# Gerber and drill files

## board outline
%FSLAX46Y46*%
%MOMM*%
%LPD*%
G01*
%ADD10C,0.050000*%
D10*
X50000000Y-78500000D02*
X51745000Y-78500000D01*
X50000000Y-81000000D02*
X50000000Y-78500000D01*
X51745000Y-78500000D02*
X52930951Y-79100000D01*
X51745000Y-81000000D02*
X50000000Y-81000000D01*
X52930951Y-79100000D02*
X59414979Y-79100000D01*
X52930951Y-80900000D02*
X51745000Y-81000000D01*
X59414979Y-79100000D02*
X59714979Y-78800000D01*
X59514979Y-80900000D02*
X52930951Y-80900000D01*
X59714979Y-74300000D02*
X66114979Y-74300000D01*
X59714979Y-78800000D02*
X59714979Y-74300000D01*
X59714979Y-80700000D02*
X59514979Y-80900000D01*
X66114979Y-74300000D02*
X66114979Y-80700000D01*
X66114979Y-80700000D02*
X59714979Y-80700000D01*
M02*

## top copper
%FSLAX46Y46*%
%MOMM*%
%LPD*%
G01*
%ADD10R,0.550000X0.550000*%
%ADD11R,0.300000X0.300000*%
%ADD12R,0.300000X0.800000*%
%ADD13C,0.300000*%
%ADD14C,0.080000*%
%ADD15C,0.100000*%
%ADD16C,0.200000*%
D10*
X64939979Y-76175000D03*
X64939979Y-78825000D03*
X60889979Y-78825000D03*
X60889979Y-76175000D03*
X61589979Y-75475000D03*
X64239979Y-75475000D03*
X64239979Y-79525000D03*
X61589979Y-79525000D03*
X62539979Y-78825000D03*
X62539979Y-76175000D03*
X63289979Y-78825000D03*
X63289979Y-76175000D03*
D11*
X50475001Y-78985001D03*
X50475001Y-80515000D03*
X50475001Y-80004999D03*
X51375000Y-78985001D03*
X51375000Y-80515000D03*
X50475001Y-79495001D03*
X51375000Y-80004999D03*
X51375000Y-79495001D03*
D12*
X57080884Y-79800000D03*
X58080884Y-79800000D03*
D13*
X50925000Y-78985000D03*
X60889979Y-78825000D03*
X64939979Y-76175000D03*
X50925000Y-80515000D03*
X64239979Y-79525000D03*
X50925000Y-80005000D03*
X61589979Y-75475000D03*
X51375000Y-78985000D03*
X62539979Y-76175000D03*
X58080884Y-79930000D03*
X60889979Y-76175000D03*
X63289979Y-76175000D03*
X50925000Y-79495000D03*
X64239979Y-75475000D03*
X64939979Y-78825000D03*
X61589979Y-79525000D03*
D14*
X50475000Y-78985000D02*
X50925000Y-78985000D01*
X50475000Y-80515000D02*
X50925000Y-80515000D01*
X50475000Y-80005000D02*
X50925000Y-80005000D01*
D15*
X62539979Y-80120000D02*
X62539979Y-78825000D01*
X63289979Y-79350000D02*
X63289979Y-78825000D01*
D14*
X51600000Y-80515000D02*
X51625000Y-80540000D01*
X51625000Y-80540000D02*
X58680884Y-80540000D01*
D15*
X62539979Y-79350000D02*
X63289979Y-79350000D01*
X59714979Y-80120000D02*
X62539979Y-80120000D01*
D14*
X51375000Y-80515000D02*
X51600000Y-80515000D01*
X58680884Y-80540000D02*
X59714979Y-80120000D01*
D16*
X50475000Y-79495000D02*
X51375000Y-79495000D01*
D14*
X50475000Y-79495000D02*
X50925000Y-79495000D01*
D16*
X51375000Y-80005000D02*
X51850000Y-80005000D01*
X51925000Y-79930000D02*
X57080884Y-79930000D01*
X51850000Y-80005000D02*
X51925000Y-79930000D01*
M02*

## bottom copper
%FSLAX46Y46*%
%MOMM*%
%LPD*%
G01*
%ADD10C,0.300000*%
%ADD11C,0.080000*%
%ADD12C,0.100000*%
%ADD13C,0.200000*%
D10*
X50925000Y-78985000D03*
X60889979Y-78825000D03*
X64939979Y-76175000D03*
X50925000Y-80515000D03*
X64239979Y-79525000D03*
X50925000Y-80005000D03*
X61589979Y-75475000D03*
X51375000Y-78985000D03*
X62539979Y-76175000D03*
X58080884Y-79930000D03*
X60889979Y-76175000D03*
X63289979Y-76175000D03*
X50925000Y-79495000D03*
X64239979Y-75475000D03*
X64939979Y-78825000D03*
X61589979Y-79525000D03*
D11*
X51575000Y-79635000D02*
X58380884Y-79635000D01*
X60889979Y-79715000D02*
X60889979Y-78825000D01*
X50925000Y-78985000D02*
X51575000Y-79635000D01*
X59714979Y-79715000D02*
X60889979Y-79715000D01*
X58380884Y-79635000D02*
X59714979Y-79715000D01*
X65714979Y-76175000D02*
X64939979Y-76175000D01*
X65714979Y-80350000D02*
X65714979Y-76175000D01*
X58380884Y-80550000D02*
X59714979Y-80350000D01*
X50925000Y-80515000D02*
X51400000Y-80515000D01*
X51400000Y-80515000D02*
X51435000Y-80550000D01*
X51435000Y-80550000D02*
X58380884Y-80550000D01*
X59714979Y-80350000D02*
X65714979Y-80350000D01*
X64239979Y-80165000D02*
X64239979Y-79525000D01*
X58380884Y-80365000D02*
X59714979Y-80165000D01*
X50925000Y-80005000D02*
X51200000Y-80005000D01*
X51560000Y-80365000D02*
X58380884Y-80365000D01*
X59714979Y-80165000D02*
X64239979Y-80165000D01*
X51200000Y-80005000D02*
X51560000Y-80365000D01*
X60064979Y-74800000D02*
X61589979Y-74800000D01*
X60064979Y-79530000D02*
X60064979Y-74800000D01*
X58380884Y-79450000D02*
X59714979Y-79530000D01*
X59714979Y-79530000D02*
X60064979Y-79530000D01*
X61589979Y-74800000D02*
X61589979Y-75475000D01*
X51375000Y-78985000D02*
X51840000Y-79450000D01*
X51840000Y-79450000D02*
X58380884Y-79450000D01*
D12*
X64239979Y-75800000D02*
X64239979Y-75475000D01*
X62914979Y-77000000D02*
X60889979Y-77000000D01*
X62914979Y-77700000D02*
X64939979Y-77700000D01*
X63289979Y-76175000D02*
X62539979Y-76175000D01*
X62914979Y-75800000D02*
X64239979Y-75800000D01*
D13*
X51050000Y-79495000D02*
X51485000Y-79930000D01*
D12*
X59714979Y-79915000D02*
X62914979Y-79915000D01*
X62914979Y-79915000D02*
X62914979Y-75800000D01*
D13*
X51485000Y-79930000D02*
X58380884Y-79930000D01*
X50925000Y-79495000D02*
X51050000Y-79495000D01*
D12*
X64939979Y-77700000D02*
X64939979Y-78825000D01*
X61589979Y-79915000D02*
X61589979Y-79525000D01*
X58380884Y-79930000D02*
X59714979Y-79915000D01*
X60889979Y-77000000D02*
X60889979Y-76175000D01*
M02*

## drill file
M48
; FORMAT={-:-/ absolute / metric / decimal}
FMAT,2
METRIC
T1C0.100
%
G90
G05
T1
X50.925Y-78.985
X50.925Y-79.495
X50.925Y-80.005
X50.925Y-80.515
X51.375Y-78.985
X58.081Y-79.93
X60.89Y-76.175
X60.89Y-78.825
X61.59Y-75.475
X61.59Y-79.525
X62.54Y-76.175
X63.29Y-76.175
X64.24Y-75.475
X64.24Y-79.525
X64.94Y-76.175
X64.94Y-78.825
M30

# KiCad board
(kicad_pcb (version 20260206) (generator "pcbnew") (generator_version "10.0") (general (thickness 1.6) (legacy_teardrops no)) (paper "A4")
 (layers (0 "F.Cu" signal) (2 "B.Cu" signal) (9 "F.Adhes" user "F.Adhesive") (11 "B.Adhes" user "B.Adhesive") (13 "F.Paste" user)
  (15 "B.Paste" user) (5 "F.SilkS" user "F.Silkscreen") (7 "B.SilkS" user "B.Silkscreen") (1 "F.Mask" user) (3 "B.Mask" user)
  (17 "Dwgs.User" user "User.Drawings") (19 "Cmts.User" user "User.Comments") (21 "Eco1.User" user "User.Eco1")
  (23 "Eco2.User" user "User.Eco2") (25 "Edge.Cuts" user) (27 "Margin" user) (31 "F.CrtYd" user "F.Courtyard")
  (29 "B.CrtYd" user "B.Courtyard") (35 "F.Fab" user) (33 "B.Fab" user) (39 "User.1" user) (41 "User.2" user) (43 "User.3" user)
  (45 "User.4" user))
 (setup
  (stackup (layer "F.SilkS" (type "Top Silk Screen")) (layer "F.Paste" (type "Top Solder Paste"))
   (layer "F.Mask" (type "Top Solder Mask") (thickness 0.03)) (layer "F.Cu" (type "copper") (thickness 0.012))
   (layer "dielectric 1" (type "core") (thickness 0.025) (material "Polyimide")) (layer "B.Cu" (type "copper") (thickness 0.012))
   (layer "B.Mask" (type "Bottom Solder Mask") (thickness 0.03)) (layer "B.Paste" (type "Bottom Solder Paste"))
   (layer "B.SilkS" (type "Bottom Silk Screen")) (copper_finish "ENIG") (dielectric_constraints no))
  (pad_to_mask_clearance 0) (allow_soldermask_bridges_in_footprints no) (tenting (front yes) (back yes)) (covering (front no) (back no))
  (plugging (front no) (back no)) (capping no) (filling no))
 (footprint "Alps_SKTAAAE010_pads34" (layer "F.Cu") (at 65.314979 77.5 -90)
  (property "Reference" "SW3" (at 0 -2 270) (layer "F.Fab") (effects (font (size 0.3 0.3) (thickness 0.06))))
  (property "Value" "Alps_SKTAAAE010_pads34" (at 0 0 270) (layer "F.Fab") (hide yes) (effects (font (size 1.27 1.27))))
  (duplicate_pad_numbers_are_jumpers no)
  (pad "3" smd rect (at -1.325 0.375 270) (size 0.55 0.55) (layers "F.Cu" "F.Mask") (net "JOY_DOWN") (solder_mask_margin 0.05)
   (thermal_bridge_angle 45))
  (pad "4" smd rect (at 1.325 0.375 270) (size 0.55 0.55) (layers "F.Cu" "F.Mask") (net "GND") (solder_mask_margin 0.05)
   (thermal_bridge_angle 45)))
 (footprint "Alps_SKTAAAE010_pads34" (layer "F.Cu") (at 62.914979 79.9 180)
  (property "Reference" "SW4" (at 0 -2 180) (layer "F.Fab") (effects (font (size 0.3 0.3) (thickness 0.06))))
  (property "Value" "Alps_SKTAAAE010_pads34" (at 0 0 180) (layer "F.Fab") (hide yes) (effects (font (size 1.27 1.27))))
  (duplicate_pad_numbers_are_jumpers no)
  (pad "3" smd rect (at -1.325 0.375 180) (size 0.55 0.55) (layers "F.Cu" "F.Mask") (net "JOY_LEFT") (solder_mask_margin 0.05)
   (thermal_bridge_angle 45))
  (pad "4" smd rect (at 1.325 0.375 180) (size 0.55 0.55) (layers "F.Cu" "F.Mask") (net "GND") (solder_mask_margin 0.05)
   (thermal_bridge_angle 45)))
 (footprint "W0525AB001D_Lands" (layer "F.Cu") (at 57.580884 79.93)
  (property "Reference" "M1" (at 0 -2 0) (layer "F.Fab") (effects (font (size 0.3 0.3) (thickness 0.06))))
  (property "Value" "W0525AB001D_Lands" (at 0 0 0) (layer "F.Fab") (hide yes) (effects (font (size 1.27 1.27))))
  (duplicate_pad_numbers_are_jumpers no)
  (pad "1" smd rect (at -0.5 -0.13) (size 0.3 0.8) (layers "F.Cu" "F.Mask") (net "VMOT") (solder_mask_margin 0.05) (thermal_bridge_angle 45))
  (pad "2" smd rect (at 0.5 -0.13) (size 0.3 0.8) (layers "F.Cu" "F.Mask") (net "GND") (solder_mask_margin 0.05) (thermal_bridge_angle 45)))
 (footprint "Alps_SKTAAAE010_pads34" (layer "F.Cu") (at 60.514979 77.5 90)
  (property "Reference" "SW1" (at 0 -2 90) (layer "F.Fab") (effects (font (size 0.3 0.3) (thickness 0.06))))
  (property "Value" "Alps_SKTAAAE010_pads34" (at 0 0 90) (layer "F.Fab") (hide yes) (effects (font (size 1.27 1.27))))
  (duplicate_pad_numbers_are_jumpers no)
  (pad "3" smd rect (at -1.325 0.375 90) (size 0.55 0.55) (layers "F.Cu" "F.Mask") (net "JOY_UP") (solder_mask_margin 0.05)
   (thermal_bridge_angle 45))
  (pad "4" smd rect (at 1.325 0.375 90) (size 0.55 0.55) (layers "F.Cu" "F.Mask") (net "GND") (solder_mask_margin 0.05)
   (thermal_bridge_angle 45)))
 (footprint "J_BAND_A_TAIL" (layer "F.Cu") (at 50.9 79.75)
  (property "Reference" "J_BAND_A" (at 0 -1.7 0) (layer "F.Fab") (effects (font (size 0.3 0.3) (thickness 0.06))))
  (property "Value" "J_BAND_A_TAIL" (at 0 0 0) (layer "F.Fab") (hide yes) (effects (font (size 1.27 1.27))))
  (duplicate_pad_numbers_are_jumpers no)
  (pad "1" smd rect (at -0.424999 -0.764999) (size 0.3 0.3) (layers "F.Cu" "F.Mask") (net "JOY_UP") (solder_mask_margin 0.05)
   (thermal_bridge_angle 45))
  (pad "2" smd rect (at -0.424999 0.765) (size 0.3 0.3) (layers "F.Cu" "F.Mask") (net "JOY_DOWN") (solder_mask_margin 0.05)
   (thermal_bridge_angle 45))
  (pad "3" smd rect (at -0.424999 0.254999) (size 0.3 0.3) (layers "F.Cu" "F.Mask") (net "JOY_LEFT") (solder_mask_margin 0.05)
   (thermal_bridge_angle 45))
  (pad "4" smd rect (at 0.475 -0.764999) (size 0.3 0.3) (layers "F.Cu" "F.Mask") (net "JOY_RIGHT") (solder_mask_margin 0.05)
   (thermal_bridge_angle 45))
  (pad "5" smd rect (at 0.475 0.765) (size 0.3 0.3) (layers "F.Cu" "F.Mask") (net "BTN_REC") (solder_mask_margin 0.05)
   (thermal_bridge_angle 45))
  (pad "6" smd rect (at -0.424999 -0.254999) (size 0.3 0.3) (layers "F.Cu" "F.Mask") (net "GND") (solder_mask_margin 0.05)
   (thermal_bridge_angle 45))
  (pad "7" smd rect (at 0.475 0.254999) (size 0.3 0.3) (layers "F.Cu" "F.Mask") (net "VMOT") (solder_mask_margin 0.05)
   (thermal_bridge_angle 45))
  (pad "8" smd rect (at 0.475 -0.254999) (size 0.3 0.3) (layers "F.Cu" "F.Mask") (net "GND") (solder_mask_margin 0.05)
   (thermal_bridge_angle 45)))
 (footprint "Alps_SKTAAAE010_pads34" (layer "F.Cu") (at 62.914979 75.1)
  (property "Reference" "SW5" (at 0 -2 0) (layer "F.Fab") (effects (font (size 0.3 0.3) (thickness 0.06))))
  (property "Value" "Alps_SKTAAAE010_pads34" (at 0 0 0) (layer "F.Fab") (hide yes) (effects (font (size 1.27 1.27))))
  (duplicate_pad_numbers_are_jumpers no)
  (pad "3" smd rect (at -1.325 0.375) (size 0.55 0.55) (layers "F.Cu" "F.Mask") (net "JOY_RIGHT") (solder_mask_margin 0.05)
   (thermal_bridge_angle 45))
  (pad "4" smd rect (at 1.325 0.375) (size 0.55 0.55) (layers "F.Cu" "F.Mask") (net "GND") (solder_mask_margin 0.05)
   (thermal_bridge_angle 45)))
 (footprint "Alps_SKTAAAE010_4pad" (layer "F.Cu") (at 62.914979 77.5 90)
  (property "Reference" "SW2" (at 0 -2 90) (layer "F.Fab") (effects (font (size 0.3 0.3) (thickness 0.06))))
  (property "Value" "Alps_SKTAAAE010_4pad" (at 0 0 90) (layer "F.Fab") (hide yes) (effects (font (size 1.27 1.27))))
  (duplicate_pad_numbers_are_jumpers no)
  (pad "1" smd rect (at -1.325 -0.375 90) (size 0.55 0.55) (layers "F.Cu" "F.Mask") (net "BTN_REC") (solder_mask_margin 0.05)
   (thermal_bridge_angle 45))
  (pad "2" smd rect (at 1.325 -0.375 90) (size 0.55 0.55) (layers "F.Cu" "F.Mask") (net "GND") (solder_mask_margin 0.05)
   (thermal_bridge_angle 45))
  (pad "3" smd rect (at -1.325 0.375 90) (size 0.55 0.55) (layers "F.Cu" "F.Mask") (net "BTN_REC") (solder_mask_margin 0.05)
   (thermal_bridge_angle 45))
  (pad "4" smd rect (at 1.325 0.375 90) (size 0.55 0.55) (layers "F.Cu" "F.Mask") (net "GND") (solder_mask_margin 0.05)
   (thermal_bridge_angle 45)))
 (gr_line (start 50 78.5) (end 51.745 78.5) (stroke (width 0.05) (type default)) (layer "Edge.Cuts"))
 (gr_line (start 50 81) (end 50 78.5) (stroke (width 0.05) (type default)) (layer "Edge.Cuts"))
 (gr_line (start 51.745 78.5) (end 52.930951 79.1) (stroke (width 0.05) (type default)) (layer "Edge.Cuts"))
 (gr_line (start 51.745 81) (end 50 81) (stroke (width 0.05) (type default)) (layer "Edge.Cuts"))
 (gr_line (start 52.930951 79.1) (end 59.414979 79.1) (stroke (width 0.05) (type default)) (layer "Edge.Cuts"))
 (gr_line (start 52.930951 80.9) (end 51.745 81) (stroke (width 0.05) (type default)) (layer "Edge.Cuts"))
 (gr_line (start 59.414979 79.1) (end 59.714979 78.8) (stroke (width 0.05) (type default)) (layer "Edge.Cuts"))
 (gr_line (start 59.514979 80.9) (end 52.930951 80.9) (stroke (width 0.05) (type default)) (layer "Edge.Cuts"))
 (gr_line (start 59.714979 74.3) (end 66.114979 74.3) (stroke (width 0.05) (type default)) (layer "Edge.Cuts"))
 (gr_line (start 59.714979 78.8) (end 59.714979 74.3) (stroke (width 0.05) (type default)) (layer "Edge.Cuts"))
 (gr_line (start 59.714979 80.7) (end 59.514979 80.9) (stroke (width 0.05) (type default)) (layer "Edge.Cuts"))
 (gr_line (start 66.114979 74.3) (end 66.114979 80.7) (stroke (width 0.05) (type default)) (layer "Edge.Cuts"))
 (gr_line (start 66.114979 80.7) (end 59.714979 80.7) (stroke (width 0.05) (type default)) (layer "Edge.Cuts"))
 (segment (start 50.475 78.985) (end 50.925 78.985) (width 0.08) (layer "F.Cu") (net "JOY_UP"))
 (via (at 60.889979 78.825) (size 0.3) (drill 0.1) (layers "F.Cu" "B.Cu") (tenting (front yes) (back yes)) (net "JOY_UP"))
 (via (at 50.925 78.985) (size 0.3) (drill 0.1) (layers "F.Cu" "B.Cu") (tenting (front yes) (back yes)) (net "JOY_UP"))
 (segment (start 60.889979 79.715) (end 60.889979 78.825) (width 0.08) (layer "B.Cu") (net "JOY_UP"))
 (segment (start 58.380884 79.635) (end 59.714979 79.715) (width 0.08) (layer "B.Cu") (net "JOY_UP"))
 (segment (start 50.925 78.985) (end 51.575 79.635) (width 0.08) (layer "B.Cu") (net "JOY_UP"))
 (segment (start 59.714979 79.715) (end 60.889979 79.715) (width 0.08) (layer "B.Cu") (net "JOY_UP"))
 (segment (start 51.575 79.635) (end 58.380884 79.635) (width 0.08) (layer "B.Cu") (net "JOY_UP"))
 (segment (start 50.475 80.515) (end 50.925 80.515) (width 0.08) (layer "F.Cu") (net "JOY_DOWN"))
 (via (at 50.925 80.515) (size 0.3) (drill 0.1) (layers "F.Cu" "B.Cu") (tenting (front yes) (back yes)) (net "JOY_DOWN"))
 (via (at 64.939979 76.175) (size 0.3) (drill 0.1) (layers "F.Cu" "B.Cu") (tenting (front yes) (back yes)) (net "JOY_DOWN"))
 (segment (start 65.714979 76.175) (end 64.939979 76.175) (width 0.08) (layer "B.Cu") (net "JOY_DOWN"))
 (segment (start 50.925 80.515) (end 51.4 80.515) (width 0.08) (layer "B.Cu") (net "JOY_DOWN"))
 (segment (start 65.714979 80.35) (end 65.714979 76.175) (width 0.08) (layer "B.Cu") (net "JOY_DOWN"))
 (segment (start 51.4 80.515) (end 51.435 80.55) (width 0.08) (layer "B.Cu") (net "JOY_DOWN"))
 (segment (start 51.435 80.55) (end 58.380884 80.55) (width 0.08) (layer "B.Cu") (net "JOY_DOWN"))
 (segment (start 58.380884 80.55) (end 59.714979 80.35) (width 0.08) (layer "B.Cu") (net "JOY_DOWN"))
 (segment (start 59.714979 80.35) (end 65.714979 80.35) (width 0.08) (layer "B.Cu") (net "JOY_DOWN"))
 (segment (start 50.475 80.005) (end 50.925 80.005) (width 0.08) (layer "F.Cu") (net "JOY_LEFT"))
 (via (at 50.925 80.005) (size 0.3) (drill 0.1) (layers "F.Cu" "B.Cu") (tenting (front yes) (back yes)) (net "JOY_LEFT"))
 (via (at 64.239979 79.525) (size 0.3) (drill 0.1) (layers "F.Cu" "B.Cu") (tenting (front yes) (back yes)) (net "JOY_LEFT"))
 (segment (start 51.2 80.005) (end 51.56 80.365) (width 0.08) (layer "B.Cu") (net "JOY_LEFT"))
 (segment (start 58.380884 80.365) (end 59.714979 80.165) (width 0.08) (layer "B.Cu") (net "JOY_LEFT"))
 (segment (start 59.714979 80.165) (end 64.239979 80.165) (width 0.08) (layer "B.Cu") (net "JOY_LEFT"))
 (segment (start 50.925 80.005) (end 51.2 80.005) (width 0.08) (layer "B.Cu") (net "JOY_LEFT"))
 (segment (start 51.56 80.365) (end 58.380884 80.365) (width 0.08) (layer "B.Cu") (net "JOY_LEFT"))
 (segment (start 64.239979 80.165) (end 64.239979 79.525) (width 0.08) (layer "B.Cu") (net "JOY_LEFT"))
 (via (at 61.589979 75.475) (size 0.3) (drill 0.1) (layers "F.Cu" "B.Cu") (tenting (front yes) (back yes)) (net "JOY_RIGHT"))
 (via (at 51.375 78.985) (size 0.3) (drill 0.1) (layers "F.Cu" "B.Cu") (tenting (front yes) (back yes)) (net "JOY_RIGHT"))
 (segment (start 61.589979 74.8) (end 61.589979 75.475) (width 0.08) (layer "B.Cu") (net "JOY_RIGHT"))
 (segment (start 51.84 79.45) (end 58.380884 79.45) (width 0.08) (layer "B.Cu") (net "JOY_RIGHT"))
 (segment (start 58.380884 79.45) (end 59.714979 79.53) (width 0.08) (layer "B.Cu") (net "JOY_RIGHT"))
 (segment (start 60.064979 79.53) (end 60.064979 74.8) (width 0.08) (layer "B.Cu") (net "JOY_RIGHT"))
 (segment (start 51.375 78.985) (end 51.84 79.45) (width 0.08) (layer "B.Cu") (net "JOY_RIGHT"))
 (segment (start 59.714979 79.53) (end 60.064979 79.53) (width 0.08) (layer "B.Cu") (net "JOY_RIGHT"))
 (segment (start 60.064979 74.8) (end 61.589979 74.8) (width 0.08) (layer "B.Cu") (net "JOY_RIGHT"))
 (segment (start 63.289979 79.35) (end 63.289979 78.825) (width 0.1) (layer "F.Cu") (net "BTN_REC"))
 (segment (start 59.714979 80.12) (end 62.539979 80.12) (width 0.1) (layer "F.Cu") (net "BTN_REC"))
 (segment (start 62.539979 79.35) (end 63.289979 79.35) (width 0.1) (layer "F.Cu") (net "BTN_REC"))
 (segment (start 62.539979 80.12) (end 62.539979 78.825) (width 0.1) (layer "F.Cu") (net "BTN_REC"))
 (segment (start 51.625 80.54) (end 58.680884 80.54) (width 0.08) (layer "F.Cu") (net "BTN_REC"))
 (segment (start 51.375 80.515) (end 51.6 80.515) (width 0.08) (layer "F.Cu") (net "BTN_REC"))
 (segment (start 58.680884 80.54) (end 59.714979 80.12) (width 0.08) (layer "F.Cu") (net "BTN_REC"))
 (segment (start 51.6 80.515) (end 51.625 80.54) (width 0.08) (layer "F.Cu") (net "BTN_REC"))
 (segment (start 50.475 79.495) (end 51.375 79.495) (width 0.2) (layer "F.Cu") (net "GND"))
 (segment (start 50.475 79.495) (end 50.925 79.495) (width 0.08) (layer "F.Cu") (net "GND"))
 (via (at 64.239979 75.475) (size 0.3) (drill 0.1) (layers "F.Cu" "B.Cu") (tenting (front yes) (back yes)) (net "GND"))
 (via (at 60.889979 76.175) (size 0.3) (drill 0.1) (layers "F.Cu" "B.Cu") (tenting (front yes) (back yes)) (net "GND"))
 (via (at 62.539979 76.175) (size 0.3) (drill 0.1) (layers "F.Cu" "B.Cu") (tenting (front yes) (back yes)) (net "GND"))
 (via (at 64.939979 78.825) (size 0.3) (drill 0.1) (layers "F.Cu" "B.Cu") (tenting (front yes) (back yes)) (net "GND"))
 (via (at 63.289979 76.175) (size 0.3) (drill 0.1) (layers "F.Cu" "B.Cu") (tenting (front yes) (back yes)) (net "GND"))
 (via (at 58.080884 79.93) (size 0.3) (drill 0.1) (layers "F.Cu" "B.Cu") (tenting (front yes) (back yes)) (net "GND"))
 (via (at 50.925 79.495) (size 0.3) (drill 0.1) (layers "F.Cu" "B.Cu") (tenting (front yes) (back yes)) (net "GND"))
 (via (at 61.589979 79.525) (size 0.3) (drill 0.1) (layers "F.Cu" "B.Cu") (tenting (front yes) (back yes)) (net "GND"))
 (segment (start 51.05 79.495) (end 51.485 79.93) (width 0.2) (layer "B.Cu") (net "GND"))
 (segment (start 60.889979 77) (end 60.889979 76.175) (width 0.1) (layer "B.Cu") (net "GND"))
 (segment (start 62.914979 77) (end 60.889979 77) (width 0.1) (layer "B.Cu") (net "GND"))
 (segment (start 50.925 79.495) (end 51.05 79.495) (width 0.2) (layer "B.Cu") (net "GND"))
 (segment (start 59.714979 79.915) (end 62.914979 79.915) (width 0.1) (layer "B.Cu") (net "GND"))
 (segment (start 64.939979 77.7) (end 64.939979 78.825) (width 0.1) (layer "B.Cu") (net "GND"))
 (segment (start 62.914979 77.7) (end 64.939979 77.7) (width 0.1) (layer "B.Cu") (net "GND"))
 (segment (start 58.380884 79.93) (end 59.714979 79.915) (width 0.1) (layer "B.Cu") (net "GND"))
 (segment (start 61.589979 79.915) (end 61.589979 79.525) (width 0.1) (layer "B.Cu") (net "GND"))
 (segment (start 63.289979 76.175) (end 62.539979 76.175) (width 0.1) (layer "B.Cu") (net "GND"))
 (segment (start 51.485 79.93) (end 58.380884 79.93) (width 0.2) (layer "B.Cu") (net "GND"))
 (segment (start 62.914979 75.8) (end 64.239979 75.8) (width 0.1) (layer "B.Cu") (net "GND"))
 (segment (start 62.914979 79.915) (end 62.914979 75.8) (width 0.1) (layer "B.Cu") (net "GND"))
 (segment (start 64.239979 75.8) (end 64.239979 75.475) (width 0.1) (layer "B.Cu") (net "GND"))
 (segment (start 51.925 79.93) (end 57.080884 79.93) (width 0.2) (layer "F.Cu") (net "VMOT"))
 (segment (start 51.375 80.005) (end 51.85 80.005) (width 0.2) (layer "F.Cu") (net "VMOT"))
 (segment (start 51.85 80.005) (end 51.925 79.93) (width 0.2) (layer "F.Cu") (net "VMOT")))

